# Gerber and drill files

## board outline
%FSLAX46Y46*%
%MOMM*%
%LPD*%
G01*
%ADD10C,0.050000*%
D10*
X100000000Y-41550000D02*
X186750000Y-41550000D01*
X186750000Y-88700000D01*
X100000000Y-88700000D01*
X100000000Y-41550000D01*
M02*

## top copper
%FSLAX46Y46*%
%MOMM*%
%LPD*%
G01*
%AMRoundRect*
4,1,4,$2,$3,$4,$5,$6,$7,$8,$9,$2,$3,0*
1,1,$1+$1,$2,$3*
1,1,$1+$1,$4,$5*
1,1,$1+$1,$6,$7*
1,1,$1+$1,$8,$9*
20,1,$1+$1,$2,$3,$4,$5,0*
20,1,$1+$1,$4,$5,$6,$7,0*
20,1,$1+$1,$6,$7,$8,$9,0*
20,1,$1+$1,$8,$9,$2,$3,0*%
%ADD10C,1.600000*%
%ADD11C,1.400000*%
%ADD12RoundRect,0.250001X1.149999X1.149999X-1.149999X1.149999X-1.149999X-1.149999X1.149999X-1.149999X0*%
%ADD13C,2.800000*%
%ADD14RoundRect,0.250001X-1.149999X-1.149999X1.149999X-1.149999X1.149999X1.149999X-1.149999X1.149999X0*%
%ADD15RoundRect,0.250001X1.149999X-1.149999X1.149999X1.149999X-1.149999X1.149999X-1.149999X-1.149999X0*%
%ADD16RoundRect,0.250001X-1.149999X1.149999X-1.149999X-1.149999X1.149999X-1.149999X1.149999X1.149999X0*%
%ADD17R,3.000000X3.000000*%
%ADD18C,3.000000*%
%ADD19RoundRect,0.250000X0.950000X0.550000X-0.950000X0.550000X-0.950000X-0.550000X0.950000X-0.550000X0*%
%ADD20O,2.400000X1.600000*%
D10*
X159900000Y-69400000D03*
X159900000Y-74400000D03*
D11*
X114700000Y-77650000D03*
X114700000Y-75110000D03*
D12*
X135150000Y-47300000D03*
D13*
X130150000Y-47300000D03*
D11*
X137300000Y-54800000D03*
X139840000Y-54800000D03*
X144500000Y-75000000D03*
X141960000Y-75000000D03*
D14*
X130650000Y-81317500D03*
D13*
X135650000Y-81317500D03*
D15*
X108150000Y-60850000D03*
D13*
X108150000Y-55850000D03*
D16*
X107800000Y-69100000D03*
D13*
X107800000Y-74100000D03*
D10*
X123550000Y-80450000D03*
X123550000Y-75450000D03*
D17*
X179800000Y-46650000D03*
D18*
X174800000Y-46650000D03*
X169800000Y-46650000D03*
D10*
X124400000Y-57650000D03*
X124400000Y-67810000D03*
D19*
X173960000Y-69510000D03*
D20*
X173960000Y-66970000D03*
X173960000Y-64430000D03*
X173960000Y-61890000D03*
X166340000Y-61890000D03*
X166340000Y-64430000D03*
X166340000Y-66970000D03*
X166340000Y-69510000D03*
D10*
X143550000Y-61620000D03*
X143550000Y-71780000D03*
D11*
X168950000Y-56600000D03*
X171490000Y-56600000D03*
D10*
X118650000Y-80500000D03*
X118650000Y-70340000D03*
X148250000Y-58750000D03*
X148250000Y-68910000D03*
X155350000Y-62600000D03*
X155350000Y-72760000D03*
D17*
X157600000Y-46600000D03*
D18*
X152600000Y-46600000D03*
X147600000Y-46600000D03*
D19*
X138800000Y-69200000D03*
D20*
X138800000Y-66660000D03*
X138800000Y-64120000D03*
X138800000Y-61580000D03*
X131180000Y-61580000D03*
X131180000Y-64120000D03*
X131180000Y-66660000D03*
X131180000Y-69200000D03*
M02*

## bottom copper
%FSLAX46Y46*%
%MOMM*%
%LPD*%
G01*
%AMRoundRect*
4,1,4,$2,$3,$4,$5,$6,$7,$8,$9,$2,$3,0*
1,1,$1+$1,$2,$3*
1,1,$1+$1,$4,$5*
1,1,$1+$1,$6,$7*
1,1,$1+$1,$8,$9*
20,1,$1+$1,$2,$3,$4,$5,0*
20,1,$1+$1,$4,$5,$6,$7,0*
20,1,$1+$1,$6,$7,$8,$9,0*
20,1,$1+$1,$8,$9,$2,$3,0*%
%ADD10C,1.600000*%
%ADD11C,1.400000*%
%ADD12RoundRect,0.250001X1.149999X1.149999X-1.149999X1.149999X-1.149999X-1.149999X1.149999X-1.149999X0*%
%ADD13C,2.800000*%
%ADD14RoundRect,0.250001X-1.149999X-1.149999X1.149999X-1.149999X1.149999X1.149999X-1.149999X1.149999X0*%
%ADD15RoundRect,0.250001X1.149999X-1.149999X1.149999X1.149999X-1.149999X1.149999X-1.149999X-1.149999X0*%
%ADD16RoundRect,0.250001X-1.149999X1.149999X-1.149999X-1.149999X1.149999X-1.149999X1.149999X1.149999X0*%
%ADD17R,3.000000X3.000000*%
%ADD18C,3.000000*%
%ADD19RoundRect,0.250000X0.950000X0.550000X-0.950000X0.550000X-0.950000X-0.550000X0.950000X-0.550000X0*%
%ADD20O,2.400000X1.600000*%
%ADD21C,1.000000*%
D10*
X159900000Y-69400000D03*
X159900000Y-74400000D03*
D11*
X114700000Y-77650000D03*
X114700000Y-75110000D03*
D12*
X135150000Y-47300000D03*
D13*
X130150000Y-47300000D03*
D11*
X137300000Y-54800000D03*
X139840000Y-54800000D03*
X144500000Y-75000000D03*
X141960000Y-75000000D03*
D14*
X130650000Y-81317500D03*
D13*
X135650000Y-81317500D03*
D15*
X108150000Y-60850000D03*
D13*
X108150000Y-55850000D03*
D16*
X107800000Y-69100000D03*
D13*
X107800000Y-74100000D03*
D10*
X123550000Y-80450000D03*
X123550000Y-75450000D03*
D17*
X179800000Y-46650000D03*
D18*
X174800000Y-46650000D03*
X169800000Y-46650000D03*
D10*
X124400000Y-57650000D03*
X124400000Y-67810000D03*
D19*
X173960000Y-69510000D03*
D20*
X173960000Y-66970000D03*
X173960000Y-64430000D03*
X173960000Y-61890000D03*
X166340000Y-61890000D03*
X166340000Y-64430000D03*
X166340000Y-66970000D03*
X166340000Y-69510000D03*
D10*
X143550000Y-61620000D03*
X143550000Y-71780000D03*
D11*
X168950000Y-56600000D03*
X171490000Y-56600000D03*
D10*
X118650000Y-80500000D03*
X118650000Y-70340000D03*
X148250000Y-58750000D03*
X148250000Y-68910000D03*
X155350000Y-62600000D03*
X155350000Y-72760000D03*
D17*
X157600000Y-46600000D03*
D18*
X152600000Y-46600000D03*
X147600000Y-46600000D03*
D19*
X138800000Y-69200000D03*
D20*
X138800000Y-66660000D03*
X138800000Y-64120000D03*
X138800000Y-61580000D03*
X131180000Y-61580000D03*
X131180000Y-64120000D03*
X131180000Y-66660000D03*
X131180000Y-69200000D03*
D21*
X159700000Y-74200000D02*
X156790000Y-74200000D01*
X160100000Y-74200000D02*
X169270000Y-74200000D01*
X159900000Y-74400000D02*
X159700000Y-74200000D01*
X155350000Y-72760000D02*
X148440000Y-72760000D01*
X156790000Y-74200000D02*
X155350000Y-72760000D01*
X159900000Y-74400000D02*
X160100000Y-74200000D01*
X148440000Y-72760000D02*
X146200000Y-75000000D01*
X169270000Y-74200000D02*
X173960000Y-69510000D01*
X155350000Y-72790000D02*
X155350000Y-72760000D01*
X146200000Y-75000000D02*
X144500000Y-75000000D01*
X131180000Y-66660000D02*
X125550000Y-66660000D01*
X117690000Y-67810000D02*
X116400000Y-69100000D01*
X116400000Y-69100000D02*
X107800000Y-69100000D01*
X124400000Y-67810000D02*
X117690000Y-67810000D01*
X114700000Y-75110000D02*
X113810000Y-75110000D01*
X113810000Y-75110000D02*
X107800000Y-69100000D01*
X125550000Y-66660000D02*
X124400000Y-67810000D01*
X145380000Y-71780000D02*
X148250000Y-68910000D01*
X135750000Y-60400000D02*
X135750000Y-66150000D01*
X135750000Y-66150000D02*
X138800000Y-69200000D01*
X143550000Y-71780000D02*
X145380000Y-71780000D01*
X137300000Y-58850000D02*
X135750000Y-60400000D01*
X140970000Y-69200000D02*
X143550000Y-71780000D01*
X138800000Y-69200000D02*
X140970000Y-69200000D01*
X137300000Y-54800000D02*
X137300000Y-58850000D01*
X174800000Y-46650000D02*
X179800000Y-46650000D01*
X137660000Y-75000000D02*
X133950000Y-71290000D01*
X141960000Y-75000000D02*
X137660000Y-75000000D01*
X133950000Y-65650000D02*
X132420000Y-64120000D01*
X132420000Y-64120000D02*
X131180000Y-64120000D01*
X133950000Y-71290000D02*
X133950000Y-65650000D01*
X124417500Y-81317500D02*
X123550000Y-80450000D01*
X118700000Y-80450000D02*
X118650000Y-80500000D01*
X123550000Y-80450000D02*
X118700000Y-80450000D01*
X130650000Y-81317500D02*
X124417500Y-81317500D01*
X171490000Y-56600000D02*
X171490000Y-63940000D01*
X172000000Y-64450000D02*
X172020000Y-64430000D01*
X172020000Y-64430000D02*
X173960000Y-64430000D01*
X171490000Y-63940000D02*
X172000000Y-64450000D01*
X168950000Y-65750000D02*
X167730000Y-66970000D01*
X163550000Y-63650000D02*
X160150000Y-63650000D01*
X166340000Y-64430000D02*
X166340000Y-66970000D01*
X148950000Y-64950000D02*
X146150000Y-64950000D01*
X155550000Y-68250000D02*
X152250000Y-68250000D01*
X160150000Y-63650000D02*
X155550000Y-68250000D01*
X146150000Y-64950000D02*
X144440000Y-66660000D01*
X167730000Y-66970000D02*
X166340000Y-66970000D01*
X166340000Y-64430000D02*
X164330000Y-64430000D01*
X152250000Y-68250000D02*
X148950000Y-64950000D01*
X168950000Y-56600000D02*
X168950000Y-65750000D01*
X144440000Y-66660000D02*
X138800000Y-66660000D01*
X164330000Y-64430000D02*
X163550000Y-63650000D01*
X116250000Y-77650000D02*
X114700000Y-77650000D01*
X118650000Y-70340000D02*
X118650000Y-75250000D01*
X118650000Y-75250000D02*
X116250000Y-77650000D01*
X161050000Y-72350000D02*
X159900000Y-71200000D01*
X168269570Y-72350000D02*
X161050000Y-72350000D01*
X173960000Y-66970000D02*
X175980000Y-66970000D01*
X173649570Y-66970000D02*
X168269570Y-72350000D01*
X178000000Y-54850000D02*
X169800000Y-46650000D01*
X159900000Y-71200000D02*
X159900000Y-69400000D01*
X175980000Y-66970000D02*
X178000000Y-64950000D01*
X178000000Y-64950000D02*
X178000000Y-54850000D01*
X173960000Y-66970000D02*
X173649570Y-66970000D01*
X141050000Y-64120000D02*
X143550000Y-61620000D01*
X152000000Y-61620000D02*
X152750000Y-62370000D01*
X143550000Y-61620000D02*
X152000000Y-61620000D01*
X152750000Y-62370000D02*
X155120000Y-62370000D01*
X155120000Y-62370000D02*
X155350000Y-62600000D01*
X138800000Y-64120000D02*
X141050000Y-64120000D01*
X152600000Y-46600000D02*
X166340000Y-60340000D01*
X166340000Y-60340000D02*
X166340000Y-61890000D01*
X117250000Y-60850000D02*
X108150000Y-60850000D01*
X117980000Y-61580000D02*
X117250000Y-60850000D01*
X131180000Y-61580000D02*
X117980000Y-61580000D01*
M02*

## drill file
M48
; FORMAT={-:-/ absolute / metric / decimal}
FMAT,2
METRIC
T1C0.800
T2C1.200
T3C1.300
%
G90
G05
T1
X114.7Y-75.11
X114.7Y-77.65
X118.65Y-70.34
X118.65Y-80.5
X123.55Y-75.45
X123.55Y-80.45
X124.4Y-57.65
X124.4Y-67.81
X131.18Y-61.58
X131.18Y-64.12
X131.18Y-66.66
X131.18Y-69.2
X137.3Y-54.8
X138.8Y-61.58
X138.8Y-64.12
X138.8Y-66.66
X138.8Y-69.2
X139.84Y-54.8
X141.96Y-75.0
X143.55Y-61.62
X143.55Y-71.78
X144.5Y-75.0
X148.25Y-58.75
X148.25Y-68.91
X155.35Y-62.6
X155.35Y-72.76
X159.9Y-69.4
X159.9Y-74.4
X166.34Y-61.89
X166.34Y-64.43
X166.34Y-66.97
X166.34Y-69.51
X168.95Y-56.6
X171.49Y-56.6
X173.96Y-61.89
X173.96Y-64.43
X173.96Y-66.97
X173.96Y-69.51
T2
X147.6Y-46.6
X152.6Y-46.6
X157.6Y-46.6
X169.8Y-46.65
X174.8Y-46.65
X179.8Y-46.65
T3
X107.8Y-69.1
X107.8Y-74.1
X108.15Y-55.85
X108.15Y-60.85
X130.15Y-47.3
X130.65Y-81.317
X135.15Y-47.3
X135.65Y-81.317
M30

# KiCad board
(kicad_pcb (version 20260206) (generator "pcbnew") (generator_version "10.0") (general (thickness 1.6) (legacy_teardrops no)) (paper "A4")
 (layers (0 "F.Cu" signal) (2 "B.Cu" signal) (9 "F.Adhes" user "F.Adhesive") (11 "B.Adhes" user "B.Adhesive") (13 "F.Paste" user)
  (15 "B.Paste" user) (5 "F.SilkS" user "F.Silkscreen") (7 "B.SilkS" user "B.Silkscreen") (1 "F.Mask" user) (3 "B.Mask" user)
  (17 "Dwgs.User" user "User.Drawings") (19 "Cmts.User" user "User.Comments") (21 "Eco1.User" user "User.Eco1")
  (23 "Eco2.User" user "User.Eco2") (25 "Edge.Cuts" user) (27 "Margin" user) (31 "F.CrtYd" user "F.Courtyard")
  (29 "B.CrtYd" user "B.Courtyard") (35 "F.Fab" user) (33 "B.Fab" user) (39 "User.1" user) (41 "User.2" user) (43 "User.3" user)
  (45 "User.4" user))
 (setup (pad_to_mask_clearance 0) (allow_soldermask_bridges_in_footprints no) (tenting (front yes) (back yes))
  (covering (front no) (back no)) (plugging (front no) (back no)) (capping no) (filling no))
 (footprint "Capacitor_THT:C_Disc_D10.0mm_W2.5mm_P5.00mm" (layer "F.Cu") (at 159.9 69.4 -90)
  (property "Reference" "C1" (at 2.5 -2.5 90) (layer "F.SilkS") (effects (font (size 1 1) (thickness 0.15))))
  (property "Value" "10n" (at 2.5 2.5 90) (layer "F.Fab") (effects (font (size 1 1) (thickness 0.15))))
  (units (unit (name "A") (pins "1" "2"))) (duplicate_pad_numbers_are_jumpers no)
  (pad "1" thru_hole circle (at 0 0 270) (size 1.6 1.6) (drill 0.8) (layers "*.Cu" "*.Mask") (remove_unused_layers no) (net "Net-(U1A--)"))
  (pad "2" thru_hole circle (at 5 0 270) (size 1.6 1.6) (drill 0.8) (layers "*.Cu" "*.Mask") (remove_unused_layers no) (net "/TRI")))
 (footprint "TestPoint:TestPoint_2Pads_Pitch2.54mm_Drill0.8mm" (layer "F.Cu") (at 114.7 77.65 90)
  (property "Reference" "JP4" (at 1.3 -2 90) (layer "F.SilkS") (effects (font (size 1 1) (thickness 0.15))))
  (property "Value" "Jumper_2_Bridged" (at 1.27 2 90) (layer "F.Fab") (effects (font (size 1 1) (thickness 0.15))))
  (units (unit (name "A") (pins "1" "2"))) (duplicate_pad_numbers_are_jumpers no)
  (pad "1" thru_hole circle (at 0 0 90) (size 1.4 1.4) (drill 0.8) (layers "*.Cu" "*.Mask") (remove_unused_layers no) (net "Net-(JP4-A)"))
  (pad "2" thru_hole circle (at 2.54 0 90) (size 1.4 1.4) (drill 0.8) (layers "*.Cu" "*.Mask") (remove_unused_layers no) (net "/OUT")))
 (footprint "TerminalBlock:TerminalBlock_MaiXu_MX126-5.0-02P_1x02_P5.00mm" (layer "F.Cu") (at 135.15 47.3 180)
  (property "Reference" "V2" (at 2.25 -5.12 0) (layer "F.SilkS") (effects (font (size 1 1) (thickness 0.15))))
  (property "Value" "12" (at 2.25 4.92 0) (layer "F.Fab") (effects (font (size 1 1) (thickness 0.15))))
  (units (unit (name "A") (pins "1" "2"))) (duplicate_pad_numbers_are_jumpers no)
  (pad "1" thru_hole roundrect (at 0 0 180) (size 2.8 2.8) (drill 1.3) (layers "*.Cu" "*.Mask") (remove_unused_layers no)
   (roundrect_rratio 0.089286) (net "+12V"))
  (pad "2" thru_hole circle (at 5 0 180) (size 2.8 2.8) (drill 1.3) (layers "*.Cu" "*.Mask") (remove_unused_layers no) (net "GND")))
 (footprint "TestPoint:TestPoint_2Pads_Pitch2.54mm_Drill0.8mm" (layer "F.Cu") (at 137.3 54.8)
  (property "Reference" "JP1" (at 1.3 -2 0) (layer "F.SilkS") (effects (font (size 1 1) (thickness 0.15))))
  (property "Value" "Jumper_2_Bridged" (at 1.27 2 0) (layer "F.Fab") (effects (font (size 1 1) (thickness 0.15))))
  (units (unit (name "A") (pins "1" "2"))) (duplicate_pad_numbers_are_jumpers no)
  (pad "1" thru_hole circle (at 0 0) (size 1.4 1.4) (drill 0.8) (layers "*.Cu" "*.Mask") (remove_unused_layers no) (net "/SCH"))
  (pad "2" thru_hole circle (at 2.54 0) (size 1.4 1.4) (drill 0.8) (layers "*.Cu" "*.Mask") (remove_unused_layers no) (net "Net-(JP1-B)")))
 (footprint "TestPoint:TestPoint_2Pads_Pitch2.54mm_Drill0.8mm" (layer "F.Cu") (at 144.5 75 180)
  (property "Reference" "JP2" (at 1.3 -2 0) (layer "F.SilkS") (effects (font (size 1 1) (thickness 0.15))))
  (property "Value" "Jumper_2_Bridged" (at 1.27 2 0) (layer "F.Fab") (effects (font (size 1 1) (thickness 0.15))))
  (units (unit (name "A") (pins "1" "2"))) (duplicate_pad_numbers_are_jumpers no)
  (pad "1" thru_hole circle (at 0 0 180) (size 1.4 1.4) (drill 0.8) (layers "*.Cu" "*.Mask") (remove_unused_layers no) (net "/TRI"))
  (pad "2" thru_hole circle (at 2.54 0 180) (size 1.4 1.4) (drill 0.8) (layers "*.Cu" "*.Mask") (remove_unused_layers no)
   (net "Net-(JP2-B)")))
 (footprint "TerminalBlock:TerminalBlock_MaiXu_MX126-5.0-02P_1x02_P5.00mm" (layer "F.Cu") (at 130.65 81.3175)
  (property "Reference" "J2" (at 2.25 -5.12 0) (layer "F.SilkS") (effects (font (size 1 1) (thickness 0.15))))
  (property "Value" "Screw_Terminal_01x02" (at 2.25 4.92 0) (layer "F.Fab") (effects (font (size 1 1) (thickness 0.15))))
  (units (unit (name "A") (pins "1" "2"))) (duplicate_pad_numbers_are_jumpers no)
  (pad "1" thru_hole roundrect (at 0 0) (size 2.8 2.8) (drill 1.3) (layers "*.Cu" "*.Mask") (remove_unused_layers no)
   (roundrect_rratio 0.089286) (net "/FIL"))
  (pad "2" thru_hole circle (at 5 0) (size 2.8 2.8) (drill 1.3) (layers "*.Cu" "*.Mask") (remove_unused_layers no) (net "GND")))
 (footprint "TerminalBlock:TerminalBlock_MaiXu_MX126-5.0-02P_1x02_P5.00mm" (layer "F.Cu") (at 108.15 60.85 90)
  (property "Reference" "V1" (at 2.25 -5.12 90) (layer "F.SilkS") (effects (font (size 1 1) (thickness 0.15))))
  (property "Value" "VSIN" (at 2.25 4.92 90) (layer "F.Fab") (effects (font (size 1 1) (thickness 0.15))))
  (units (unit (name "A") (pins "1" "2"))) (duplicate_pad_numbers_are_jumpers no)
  (pad "1" thru_hole roundrect (at 0 0 90) (size 2.8 2.8) (drill 1.3) (layers "*.Cu" "*.Mask") (remove_unused_layers no)
   (roundrect_rratio 0.089286) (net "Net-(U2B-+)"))
  (pad "2" thru_hole circle (at 5 0 90) (size 2.8 2.8) (drill 1.3) (layers "*.Cu" "*.Mask") (remove_unused_layers no) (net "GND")))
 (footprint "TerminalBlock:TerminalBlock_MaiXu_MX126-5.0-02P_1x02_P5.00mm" (layer "F.Cu") (at 107.8 69.1 -90)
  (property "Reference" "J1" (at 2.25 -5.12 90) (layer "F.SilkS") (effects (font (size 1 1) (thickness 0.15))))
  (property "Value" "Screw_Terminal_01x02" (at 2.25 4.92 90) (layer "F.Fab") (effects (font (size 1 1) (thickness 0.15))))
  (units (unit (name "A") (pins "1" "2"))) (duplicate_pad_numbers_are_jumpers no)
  (pad "1" thru_hole roundrect (at 0 0 270) (size 2.8 2.8) (drill 1.3) (layers "*.Cu" "*.Mask") (remove_unused_layers no)
   (roundrect_rratio 0.089286) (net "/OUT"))
  (pad "2" thru_hole circle (at 5 0 270) (size 2.8 2.8) (drill 1.3) (layers "*.Cu" "*.Mask") (remove_unused_layers no) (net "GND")))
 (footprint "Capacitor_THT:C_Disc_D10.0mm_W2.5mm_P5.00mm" (layer "F.Cu") (at 123.55 80.45 90)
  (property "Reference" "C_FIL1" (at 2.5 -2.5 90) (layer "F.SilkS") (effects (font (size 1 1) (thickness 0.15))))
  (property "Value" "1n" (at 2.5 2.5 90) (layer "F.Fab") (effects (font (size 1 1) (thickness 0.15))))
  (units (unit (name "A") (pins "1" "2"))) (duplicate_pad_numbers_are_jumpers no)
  (pad "1" thru_hole circle (at 0 0 90) (size 1.6 1.6) (drill 0.8) (layers "*.Cu" "*.Mask") (remove_unused_layers no) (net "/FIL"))
  (pad "2" thru_hole circle (at 5 0 90) (size 1.6 1.6) (drill 0.8) (layers "*.Cu" "*.Mask") (remove_unused_layers no) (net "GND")))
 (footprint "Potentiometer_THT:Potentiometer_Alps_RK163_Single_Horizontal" (layer "F.Cu") (at 179.8 46.65 -90)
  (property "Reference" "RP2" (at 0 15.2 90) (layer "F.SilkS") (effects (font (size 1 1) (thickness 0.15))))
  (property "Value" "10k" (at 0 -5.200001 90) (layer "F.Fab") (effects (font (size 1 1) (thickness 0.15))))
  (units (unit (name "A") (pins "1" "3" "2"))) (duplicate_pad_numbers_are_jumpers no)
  (pad "1" thru_hole rect (at 0 0 90) (size 3 3) (drill 1.2) (layers "*.Cu" "*.Mask") (remove_unused_layers no) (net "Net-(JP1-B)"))
  (pad "2" thru_hole circle (at 0 5 90) (size 3 3) (drill 1.2) (layers "*.Cu" "*.Mask") (remove_unused_layers no) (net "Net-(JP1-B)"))
  (pad "3" thru_hole circle (at 0 10 90) (size 3 3) (drill 1.2) (layers "*.Cu" "*.Mask") (remove_unused_layers no) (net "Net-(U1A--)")))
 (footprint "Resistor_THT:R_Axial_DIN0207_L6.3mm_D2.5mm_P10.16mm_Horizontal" (layer "F.Cu") (at 124.4 57.65 -90)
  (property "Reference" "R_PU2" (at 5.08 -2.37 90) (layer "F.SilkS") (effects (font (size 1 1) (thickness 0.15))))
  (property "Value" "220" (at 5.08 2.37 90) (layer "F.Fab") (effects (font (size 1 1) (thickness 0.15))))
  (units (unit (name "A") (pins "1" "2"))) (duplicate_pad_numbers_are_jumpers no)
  (pad "1" thru_hole circle (at 0 0 270) (size 1.6 1.6) (drill 0.8) (layers "*.Cu" "*.Mask") (remove_unused_layers no) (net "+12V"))
  (pad "2" thru_hole circle (at 10.16 0 270) (size 1.6 1.6) (drill 0.8) (layers "*.Cu" "*.Mask") (remove_unused_layers no) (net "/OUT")))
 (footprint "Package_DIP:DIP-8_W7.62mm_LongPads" (layer "F.Cu") (at 173.96 69.51 180)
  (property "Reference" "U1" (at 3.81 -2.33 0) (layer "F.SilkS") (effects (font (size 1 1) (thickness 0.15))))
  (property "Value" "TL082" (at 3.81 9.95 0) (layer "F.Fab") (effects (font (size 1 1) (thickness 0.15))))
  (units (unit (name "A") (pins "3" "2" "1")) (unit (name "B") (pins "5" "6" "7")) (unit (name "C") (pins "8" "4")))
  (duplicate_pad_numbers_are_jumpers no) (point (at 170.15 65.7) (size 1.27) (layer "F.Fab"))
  (pad "1" thru_hole roundrect (at 0 0 180) (size 2.4 1.6) (drill 0.8) (layers "*.Cu" "*.Mask") (remove_unused_layers no)
   (roundrect_rratio 0.15625) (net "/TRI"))
  (pad "2" thru_hole oval (at 0 2.54 180) (size 2.4 1.6) (drill 0.8) (layers "*.Cu" "*.Mask") (remove_unused_layers no) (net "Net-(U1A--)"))
  (pad "3" thru_hole oval (at 0 5.08 180) (size 2.4 1.6) (drill 0.8) (layers "*.Cu" "*.Mask") (remove_unused_layers no) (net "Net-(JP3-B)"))
  (pad "4" thru_hole oval (at 0 7.62 180) (size 2.4 1.6) (drill 0.8) (layers "*.Cu" "*.Mask") (remove_unused_layers no) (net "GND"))
  (pad "5" thru_hole oval (at 7.62 7.62 180) (size 2.4 1.6) (drill 0.8) (layers "*.Cu" "*.Mask") (remove_unused_layers no)
   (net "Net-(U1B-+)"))
  (pad "6" thru_hole oval (at 7.62 5.08 180) (size 2.4 1.6) (drill 0.8) (layers "*.Cu" "*.Mask") (remove_unused_layers no) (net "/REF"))
  (pad "7" thru_hole oval (at 7.62 2.54 180) (size 2.4 1.6) (drill 0.8) (layers "*.Cu" "*.Mask") (remove_unused_layers no) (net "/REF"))
  (pad "8" thru_hole oval (at 7.62 0 180) (size 2.4 1.6) (drill 0.8) (layers "*.Cu" "*.Mask") (remove_unused_layers no) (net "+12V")))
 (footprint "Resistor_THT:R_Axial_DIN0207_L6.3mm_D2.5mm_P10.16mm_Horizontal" (layer "F.Cu") (at 143.55 61.62 -90)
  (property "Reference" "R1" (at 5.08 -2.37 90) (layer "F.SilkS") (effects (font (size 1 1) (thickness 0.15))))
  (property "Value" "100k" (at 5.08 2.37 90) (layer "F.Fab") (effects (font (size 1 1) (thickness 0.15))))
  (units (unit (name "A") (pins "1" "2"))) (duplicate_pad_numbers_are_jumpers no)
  (pad "1" thru_hole circle (at 0 0 270) (size 1.6 1.6) (drill 0.8) (layers "*.Cu" "*.Mask") (remove_unused_layers no) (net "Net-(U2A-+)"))
  (pad "2" thru_hole circle (at 10.16 0 270) (size 1.6 1.6) (drill 0.8) (layers "*.Cu" "*.Mask") (remove_unused_layers no) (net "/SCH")))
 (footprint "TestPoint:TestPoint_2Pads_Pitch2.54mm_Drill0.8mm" (layer "F.Cu") (at 168.95 56.6)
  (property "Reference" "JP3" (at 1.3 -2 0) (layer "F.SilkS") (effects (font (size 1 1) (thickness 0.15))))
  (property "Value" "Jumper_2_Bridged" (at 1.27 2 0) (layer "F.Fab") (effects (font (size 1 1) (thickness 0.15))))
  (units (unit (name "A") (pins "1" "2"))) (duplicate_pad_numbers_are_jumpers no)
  (pad "1" thru_hole circle (at 0 0) (size 1.4 1.4) (drill 0.8) (layers "*.Cu" "*.Mask") (remove_unused_layers no) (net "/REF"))
  (pad "2" thru_hole circle (at 2.54 0) (size 1.4 1.4) (drill 0.8) (layers "*.Cu" "*.Mask") (remove_unused_layers no) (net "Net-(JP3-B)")))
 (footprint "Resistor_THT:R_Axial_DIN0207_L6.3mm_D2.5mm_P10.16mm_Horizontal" (layer "F.Cu") (at 118.65 80.5 90)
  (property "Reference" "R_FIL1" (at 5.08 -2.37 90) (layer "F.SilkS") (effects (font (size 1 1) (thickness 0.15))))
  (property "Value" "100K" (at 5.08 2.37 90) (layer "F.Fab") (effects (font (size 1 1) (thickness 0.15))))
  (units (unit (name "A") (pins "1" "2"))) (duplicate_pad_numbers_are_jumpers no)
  (pad "1" thru_hole circle (at 0 0 90) (size 1.6 1.6) (drill 0.8) (layers "*.Cu" "*.Mask") (remove_unused_layers no) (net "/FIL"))
  (pad "2" thru_hole circle (at 10.16 0 90) (size 1.6 1.6) (drill 0.8) (layers "*.Cu" "*.Mask") (remove_unused_layers no)
   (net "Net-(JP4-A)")))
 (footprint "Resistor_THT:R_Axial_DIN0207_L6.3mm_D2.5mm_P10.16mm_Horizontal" (layer "F.Cu") (at 148.25 58.75 -90)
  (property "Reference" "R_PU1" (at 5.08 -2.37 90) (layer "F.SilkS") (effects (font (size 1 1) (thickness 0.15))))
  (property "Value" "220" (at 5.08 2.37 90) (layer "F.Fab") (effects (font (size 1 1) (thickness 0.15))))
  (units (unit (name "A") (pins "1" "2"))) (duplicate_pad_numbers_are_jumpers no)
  (pad "1" thru_hole circle (at 0 0 270) (size 1.6 1.6) (drill 0.8) (layers "*.Cu" "*.Mask") (remove_unused_layers no) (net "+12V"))
  (pad "2" thru_hole circle (at 10.16 0 270) (size 1.6 1.6) (drill 0.8) (layers "*.Cu" "*.Mask") (remove_unused_layers no) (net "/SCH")))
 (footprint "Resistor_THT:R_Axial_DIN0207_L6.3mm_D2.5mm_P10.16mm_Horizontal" (layer "F.Cu") (at 155.35 62.6 -90)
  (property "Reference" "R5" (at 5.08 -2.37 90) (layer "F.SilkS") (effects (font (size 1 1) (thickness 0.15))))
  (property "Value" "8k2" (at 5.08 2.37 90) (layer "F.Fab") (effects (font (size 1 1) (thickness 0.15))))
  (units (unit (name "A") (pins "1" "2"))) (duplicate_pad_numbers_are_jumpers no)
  (pad "1" thru_hole circle (at 0 0 270) (size 1.6 1.6) (drill 0.8) (layers "*.Cu" "*.Mask") (remove_unused_layers no) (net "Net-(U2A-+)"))
  (pad "2" thru_hole circle (at 10.16 0 270) (size 1.6 1.6) (drill 0.8) (layers "*.Cu" "*.Mask") (remove_unused_layers no) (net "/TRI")))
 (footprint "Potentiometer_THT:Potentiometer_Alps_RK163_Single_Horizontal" (layer "F.Cu") (at 157.6 46.6 -90)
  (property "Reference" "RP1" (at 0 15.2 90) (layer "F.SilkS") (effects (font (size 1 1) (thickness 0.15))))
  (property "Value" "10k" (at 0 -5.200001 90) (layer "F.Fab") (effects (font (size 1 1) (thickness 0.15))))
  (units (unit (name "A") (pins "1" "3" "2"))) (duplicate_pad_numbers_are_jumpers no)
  (pad "1" thru_hole rect (at 0 0 90) (size 3 3) (drill 1.2) (layers "*.Cu" "*.Mask") (remove_unused_layers no) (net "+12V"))
  (pad "2" thru_hole circle (at 0 5 90) (size 3 3) (drill 1.2) (layers "*.Cu" "*.Mask") (remove_unused_layers no) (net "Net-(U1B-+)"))
  (pad "3" thru_hole circle (at 0 10 90) (size 3 3) (drill 1.2) (layers "*.Cu" "*.Mask") (remove_unused_layers no) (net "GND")))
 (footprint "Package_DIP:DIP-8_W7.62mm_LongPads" (layer "F.Cu") (at 138.8 69.2 180)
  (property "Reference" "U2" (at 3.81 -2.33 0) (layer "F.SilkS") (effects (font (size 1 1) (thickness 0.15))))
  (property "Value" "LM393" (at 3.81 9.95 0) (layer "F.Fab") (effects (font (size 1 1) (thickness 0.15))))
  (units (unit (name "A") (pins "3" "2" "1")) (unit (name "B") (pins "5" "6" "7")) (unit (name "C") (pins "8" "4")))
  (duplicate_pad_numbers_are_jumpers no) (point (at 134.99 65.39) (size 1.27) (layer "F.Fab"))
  (pad "1" thru_hole roundrect (at 0 0 180) (size 2.4 1.6) (drill 0.8) (layers "*.Cu" "*.Mask") (remove_unused_layers no)
   (roundrect_rratio 0.15625) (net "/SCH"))
  (pad "2" thru_hole oval (at 0 2.54 180) (size 2.4 1.6) (drill 0.8) (layers "*.Cu" "*.Mask") (remove_unused_layers no) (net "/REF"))
  (pad "3" thru_hole oval (at 0 5.08 180) (size 2.4 1.6) (drill 0.8) (layers "*.Cu" "*.Mask") (remove_unused_layers no) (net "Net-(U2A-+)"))
  (pad "4" thru_hole oval (at 0 7.62 180) (size 2.4 1.6) (drill 0.8) (layers "*.Cu" "*.Mask") (remove_unused_layers no) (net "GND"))
  (pad "5" thru_hole oval (at 7.62 7.62 180) (size 2.4 1.6) (drill 0.8) (layers "*.Cu" "*.Mask") (remove_unused_layers no)
   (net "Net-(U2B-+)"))
  (pad "6" thru_hole oval (at 7.62 5.08 180) (size 2.4 1.6) (drill 0.8) (layers "*.Cu" "*.Mask") (remove_unused_layers no)
   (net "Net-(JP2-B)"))
  (pad "7" thru_hole oval (at 7.62 2.54 180) (size 2.4 1.6) (drill 0.8) (layers "*.Cu" "*.Mask") (remove_unused_layers no) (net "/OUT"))
  (pad "8" thru_hole oval (at 7.62 0 180) (size 2.4 1.6) (drill 0.8) (layers "*.Cu" "*.Mask") (remove_unused_layers no) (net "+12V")))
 (gr_rect (start 100 41.55) (end 186.75 88.7) (stroke (width 0.05) (type default)) (fill no) (layer "Edge.Cuts"))
 (segment (start 159.7 74.2) (end 156.79 74.2) (width 1) (layer "B.Cu") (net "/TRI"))
 (segment (start 160.1 74.2) (end 169.27 74.2) (width 1) (layer "B.Cu") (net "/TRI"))
 (segment (start 159.9 74.4) (end 159.7 74.2) (width 1) (layer "B.Cu") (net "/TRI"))
 (segment (start 155.35 72.76) (end 148.44 72.76) (width 1) (layer "B.Cu") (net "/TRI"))
 (segment (start 156.79 74.2) (end 155.35 72.76) (width 1) (layer "B.Cu") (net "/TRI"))
 (segment (start 159.9 74.4) (end 160.1 74.2) (width 1) (layer "B.Cu") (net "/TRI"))
 (segment (start 148.44 72.76) (end 146.2 75) (width 1) (layer "B.Cu") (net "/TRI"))
 (segment (start 169.27 74.2) (end 173.96 69.51) (width 1) (layer "B.Cu") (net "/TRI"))
 (segment (start 155.35 72.79) (end 155.35 72.76) (width 1) (layer "B.Cu") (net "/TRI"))
 (segment (start 146.2 75) (end 144.5 75) (width 1) (layer "B.Cu") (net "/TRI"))
 (segment (start 131.18 66.66) (end 125.55 66.66) (width 1) (layer "B.Cu") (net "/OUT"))
 (segment (start 117.69 67.81) (end 116.4 69.1) (width 1) (layer "B.Cu") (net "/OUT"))
 (segment (start 116.4 69.1) (end 107.8 69.1) (width 1) (layer "B.Cu") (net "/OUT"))
 (segment (start 124.4 67.81) (end 117.69 67.81) (width 1) (layer "B.Cu") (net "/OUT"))
 (segment (start 114.7 75.11) (end 113.81 75.11) (width 1) (layer "B.Cu") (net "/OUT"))
 (segment (start 113.81 75.11) (end 107.8 69.1) (width 1) (layer "B.Cu") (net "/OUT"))
 (segment (start 125.55 66.66) (end 124.4 67.81) (width 1) (layer "B.Cu") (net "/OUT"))
 (segment (start 145.38 71.78) (end 148.25 68.91) (width 1) (layer "B.Cu") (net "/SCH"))
 (segment (start 135.75 60.4) (end 135.75 66.15) (width 1) (layer "B.Cu") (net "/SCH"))
 (segment (start 135.75 66.15) (end 138.8 69.2) (width 1) (layer "B.Cu") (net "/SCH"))
 (segment (start 143.55 71.78) (end 145.38 71.78) (width 1) (layer "B.Cu") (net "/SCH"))
 (segment (start 137.3 58.85) (end 135.75 60.4) (width 1) (layer "B.Cu") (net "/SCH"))
 (segment (start 140.97 69.2) (end 143.55 71.78) (width 1) (layer "B.Cu") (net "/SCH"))
 (segment (start 138.8 69.2) (end 140.97 69.2) (width 1) (layer "B.Cu") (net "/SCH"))
 (segment (start 137.3 54.8) (end 137.3 58.85) (width 1) (layer "B.Cu") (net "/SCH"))
 (segment (start 174.8 46.65) (end 179.8 46.65) (width 1) (layer "B.Cu") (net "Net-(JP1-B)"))
 (segment (start 137.66 75) (end 133.95 71.29) (width 1) (layer "B.Cu") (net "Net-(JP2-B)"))
 (segment (start 141.96 75) (end 137.66 75) (width 1) (layer "B.Cu") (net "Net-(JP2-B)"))
 (segment (start 133.95 65.65) (end 132.42 64.12) (width 1) (layer "B.Cu") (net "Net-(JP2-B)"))
 (segment (start 132.42 64.12) (end 131.18 64.12) (width 1) (layer "B.Cu") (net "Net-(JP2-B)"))
 (segment (start 133.95 71.29) (end 133.95 65.65) (width 1) (layer "B.Cu") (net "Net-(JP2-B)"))
 (segment (start 124.4175 81.3175) (end 123.55 80.45) (width 1) (layer "B.Cu") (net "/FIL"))
 (segment (start 118.7 80.45) (end 118.65 80.5) (width 1) (layer "B.Cu") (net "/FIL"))
 (segment (start 123.55 80.45) (end 118.7 80.45) (width 1) (layer "B.Cu") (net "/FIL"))
 (segment (start 130.65 81.3175) (end 124.4175 81.3175) (width 1) (layer "B.Cu") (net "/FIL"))
 (segment (start 171.49 56.6) (end 171.49 63.94) (width 1) (layer "B.Cu") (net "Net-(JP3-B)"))
 (segment (start 172 64.45) (end 172.02 64.43) (width 1) (layer "B.Cu") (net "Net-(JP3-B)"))
 (segment (start 172.02 64.43) (end 173.96 64.43) (width 1) (layer "B.Cu") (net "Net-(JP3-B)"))
 (segment (start 171.49 63.94) (end 172 64.45) (width 1) (layer "B.Cu") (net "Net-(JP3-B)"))
 (segment (start 168.95 65.75) (end 167.73 66.97) (width 1) (layer "B.Cu") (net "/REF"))
 (segment (start 163.55 63.65) (end 160.15 63.65) (width 1) (layer "B.Cu") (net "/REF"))
 (segment (start 166.34 64.43) (end 166.34 66.97) (width 1) (layer "B.Cu") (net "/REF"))
 (segment (start 148.95 64.95) (end 146.15 64.95) (width 1) (layer "B.Cu") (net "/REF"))
 (segment (start 155.55 68.25) (end 152.25 68.25) (width 1) (layer "B.Cu") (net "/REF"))
 (segment (start 160.15 63.65) (end 155.55 68.25) (width 1) (layer "B.Cu") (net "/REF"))
 (segment (start 146.15 64.95) (end 144.44 66.66) (width 1) (layer "B.Cu") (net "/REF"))
 (segment (start 167.73 66.97) (end 166.34 66.97) (width 1) (layer "B.Cu") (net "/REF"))
 (segment (start 166.34 64.43) (end 164.33 64.43) (width 1) (layer "B.Cu") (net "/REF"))
 (segment (start 152.25 68.25) (end 148.95 64.95) (width 1) (layer "B.Cu") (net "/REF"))
 (segment (start 168.95 56.6) (end 168.95 65.75) (width 1) (layer "B.Cu") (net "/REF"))
 (segment (start 144.44 66.66) (end 138.8 66.66) (width 1) (layer "B.Cu") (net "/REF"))
 (segment (start 164.33 64.43) (end 163.55 63.65) (width 1) (layer "B.Cu") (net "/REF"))
 (segment (start 116.25 77.65) (end 114.7 77.65) (width 1) (layer "B.Cu") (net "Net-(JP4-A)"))
 (segment (start 118.65 70.34) (end 118.65 75.25) (width 1) (layer "B.Cu") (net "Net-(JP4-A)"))
 (segment (start 118.65 75.25) (end 116.25 77.65) (width 1) (layer "B.Cu") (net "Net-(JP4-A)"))
 (segment (start 161.05 72.35) (end 159.9 71.2) (width 1) (layer "B.Cu") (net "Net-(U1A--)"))
 (segment (start 168.26957 72.35) (end 161.05 72.35) (width 1) (layer "B.Cu") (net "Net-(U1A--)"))
 (segment (start 173.96 66.97) (end 175.98 66.97) (width 1) (layer "B.Cu") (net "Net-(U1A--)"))
 (segment (start 173.64957 66.97) (end 168.26957 72.35) (width 1) (layer "B.Cu") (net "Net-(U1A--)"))
 (segment (start 178 54.85) (end 169.8 46.65) (width 1) (layer "B.Cu") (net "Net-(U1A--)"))
 (segment (start 159.9 71.2) (end 159.9 69.4) (width 1) (layer "B.Cu") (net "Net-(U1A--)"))
 (segment (start 175.98 66.97) (end 178 64.95) (width 1) (layer "B.Cu") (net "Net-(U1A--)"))
 (segment (start 178 64.95) (end 178 54.85) (width 1) (layer "B.Cu") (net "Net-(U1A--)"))
 (segment (start 173.96 66.97) (end 173.64957 66.97) (width 1) (layer "B.Cu") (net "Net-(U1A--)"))
 (segment (start 141.05 64.12) (end 143.55 61.62) (width 1) (layer "B.Cu") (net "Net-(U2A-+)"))
 (segment (start 152 61.62) (end 152.75 62.37) (width 1) (layer "B.Cu") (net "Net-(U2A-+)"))
 (segment (start 143.55 61.62) (end 152 61.62) (width 1) (layer "B.Cu") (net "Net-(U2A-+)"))
 (segment (start 152.75 62.37) (end 155.12 62.37) (width 1) (layer "B.Cu") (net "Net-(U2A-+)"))
 (segment (start 155.12 62.37) (end 155.35 62.6) (width 1) (layer "B.Cu") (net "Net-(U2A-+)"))
 (segment (start 138.8 64.12) (end 141.05 64.12) (width 1) (layer "B.Cu") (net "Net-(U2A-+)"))
 (segment (start 152.6 46.6) (end 166.34 60.34) (width 1) (layer "B.Cu") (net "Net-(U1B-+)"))
 (segment (start 166.34 60.34) (end 166.34 61.89) (width 1) (layer "B.Cu") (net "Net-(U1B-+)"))
 (segment (start 117.25 60.85) (end 108.15 60.85) (width 1) (layer "B.Cu") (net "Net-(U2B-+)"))
 (segment (start 117.98 61.58) (end 117.25 60.85) (width 1) (layer "B.Cu") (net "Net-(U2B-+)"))
 (segment (start 131.18 61.58) (end 117.98 61.58) (width 1) (layer "B.Cu") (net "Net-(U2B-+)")))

